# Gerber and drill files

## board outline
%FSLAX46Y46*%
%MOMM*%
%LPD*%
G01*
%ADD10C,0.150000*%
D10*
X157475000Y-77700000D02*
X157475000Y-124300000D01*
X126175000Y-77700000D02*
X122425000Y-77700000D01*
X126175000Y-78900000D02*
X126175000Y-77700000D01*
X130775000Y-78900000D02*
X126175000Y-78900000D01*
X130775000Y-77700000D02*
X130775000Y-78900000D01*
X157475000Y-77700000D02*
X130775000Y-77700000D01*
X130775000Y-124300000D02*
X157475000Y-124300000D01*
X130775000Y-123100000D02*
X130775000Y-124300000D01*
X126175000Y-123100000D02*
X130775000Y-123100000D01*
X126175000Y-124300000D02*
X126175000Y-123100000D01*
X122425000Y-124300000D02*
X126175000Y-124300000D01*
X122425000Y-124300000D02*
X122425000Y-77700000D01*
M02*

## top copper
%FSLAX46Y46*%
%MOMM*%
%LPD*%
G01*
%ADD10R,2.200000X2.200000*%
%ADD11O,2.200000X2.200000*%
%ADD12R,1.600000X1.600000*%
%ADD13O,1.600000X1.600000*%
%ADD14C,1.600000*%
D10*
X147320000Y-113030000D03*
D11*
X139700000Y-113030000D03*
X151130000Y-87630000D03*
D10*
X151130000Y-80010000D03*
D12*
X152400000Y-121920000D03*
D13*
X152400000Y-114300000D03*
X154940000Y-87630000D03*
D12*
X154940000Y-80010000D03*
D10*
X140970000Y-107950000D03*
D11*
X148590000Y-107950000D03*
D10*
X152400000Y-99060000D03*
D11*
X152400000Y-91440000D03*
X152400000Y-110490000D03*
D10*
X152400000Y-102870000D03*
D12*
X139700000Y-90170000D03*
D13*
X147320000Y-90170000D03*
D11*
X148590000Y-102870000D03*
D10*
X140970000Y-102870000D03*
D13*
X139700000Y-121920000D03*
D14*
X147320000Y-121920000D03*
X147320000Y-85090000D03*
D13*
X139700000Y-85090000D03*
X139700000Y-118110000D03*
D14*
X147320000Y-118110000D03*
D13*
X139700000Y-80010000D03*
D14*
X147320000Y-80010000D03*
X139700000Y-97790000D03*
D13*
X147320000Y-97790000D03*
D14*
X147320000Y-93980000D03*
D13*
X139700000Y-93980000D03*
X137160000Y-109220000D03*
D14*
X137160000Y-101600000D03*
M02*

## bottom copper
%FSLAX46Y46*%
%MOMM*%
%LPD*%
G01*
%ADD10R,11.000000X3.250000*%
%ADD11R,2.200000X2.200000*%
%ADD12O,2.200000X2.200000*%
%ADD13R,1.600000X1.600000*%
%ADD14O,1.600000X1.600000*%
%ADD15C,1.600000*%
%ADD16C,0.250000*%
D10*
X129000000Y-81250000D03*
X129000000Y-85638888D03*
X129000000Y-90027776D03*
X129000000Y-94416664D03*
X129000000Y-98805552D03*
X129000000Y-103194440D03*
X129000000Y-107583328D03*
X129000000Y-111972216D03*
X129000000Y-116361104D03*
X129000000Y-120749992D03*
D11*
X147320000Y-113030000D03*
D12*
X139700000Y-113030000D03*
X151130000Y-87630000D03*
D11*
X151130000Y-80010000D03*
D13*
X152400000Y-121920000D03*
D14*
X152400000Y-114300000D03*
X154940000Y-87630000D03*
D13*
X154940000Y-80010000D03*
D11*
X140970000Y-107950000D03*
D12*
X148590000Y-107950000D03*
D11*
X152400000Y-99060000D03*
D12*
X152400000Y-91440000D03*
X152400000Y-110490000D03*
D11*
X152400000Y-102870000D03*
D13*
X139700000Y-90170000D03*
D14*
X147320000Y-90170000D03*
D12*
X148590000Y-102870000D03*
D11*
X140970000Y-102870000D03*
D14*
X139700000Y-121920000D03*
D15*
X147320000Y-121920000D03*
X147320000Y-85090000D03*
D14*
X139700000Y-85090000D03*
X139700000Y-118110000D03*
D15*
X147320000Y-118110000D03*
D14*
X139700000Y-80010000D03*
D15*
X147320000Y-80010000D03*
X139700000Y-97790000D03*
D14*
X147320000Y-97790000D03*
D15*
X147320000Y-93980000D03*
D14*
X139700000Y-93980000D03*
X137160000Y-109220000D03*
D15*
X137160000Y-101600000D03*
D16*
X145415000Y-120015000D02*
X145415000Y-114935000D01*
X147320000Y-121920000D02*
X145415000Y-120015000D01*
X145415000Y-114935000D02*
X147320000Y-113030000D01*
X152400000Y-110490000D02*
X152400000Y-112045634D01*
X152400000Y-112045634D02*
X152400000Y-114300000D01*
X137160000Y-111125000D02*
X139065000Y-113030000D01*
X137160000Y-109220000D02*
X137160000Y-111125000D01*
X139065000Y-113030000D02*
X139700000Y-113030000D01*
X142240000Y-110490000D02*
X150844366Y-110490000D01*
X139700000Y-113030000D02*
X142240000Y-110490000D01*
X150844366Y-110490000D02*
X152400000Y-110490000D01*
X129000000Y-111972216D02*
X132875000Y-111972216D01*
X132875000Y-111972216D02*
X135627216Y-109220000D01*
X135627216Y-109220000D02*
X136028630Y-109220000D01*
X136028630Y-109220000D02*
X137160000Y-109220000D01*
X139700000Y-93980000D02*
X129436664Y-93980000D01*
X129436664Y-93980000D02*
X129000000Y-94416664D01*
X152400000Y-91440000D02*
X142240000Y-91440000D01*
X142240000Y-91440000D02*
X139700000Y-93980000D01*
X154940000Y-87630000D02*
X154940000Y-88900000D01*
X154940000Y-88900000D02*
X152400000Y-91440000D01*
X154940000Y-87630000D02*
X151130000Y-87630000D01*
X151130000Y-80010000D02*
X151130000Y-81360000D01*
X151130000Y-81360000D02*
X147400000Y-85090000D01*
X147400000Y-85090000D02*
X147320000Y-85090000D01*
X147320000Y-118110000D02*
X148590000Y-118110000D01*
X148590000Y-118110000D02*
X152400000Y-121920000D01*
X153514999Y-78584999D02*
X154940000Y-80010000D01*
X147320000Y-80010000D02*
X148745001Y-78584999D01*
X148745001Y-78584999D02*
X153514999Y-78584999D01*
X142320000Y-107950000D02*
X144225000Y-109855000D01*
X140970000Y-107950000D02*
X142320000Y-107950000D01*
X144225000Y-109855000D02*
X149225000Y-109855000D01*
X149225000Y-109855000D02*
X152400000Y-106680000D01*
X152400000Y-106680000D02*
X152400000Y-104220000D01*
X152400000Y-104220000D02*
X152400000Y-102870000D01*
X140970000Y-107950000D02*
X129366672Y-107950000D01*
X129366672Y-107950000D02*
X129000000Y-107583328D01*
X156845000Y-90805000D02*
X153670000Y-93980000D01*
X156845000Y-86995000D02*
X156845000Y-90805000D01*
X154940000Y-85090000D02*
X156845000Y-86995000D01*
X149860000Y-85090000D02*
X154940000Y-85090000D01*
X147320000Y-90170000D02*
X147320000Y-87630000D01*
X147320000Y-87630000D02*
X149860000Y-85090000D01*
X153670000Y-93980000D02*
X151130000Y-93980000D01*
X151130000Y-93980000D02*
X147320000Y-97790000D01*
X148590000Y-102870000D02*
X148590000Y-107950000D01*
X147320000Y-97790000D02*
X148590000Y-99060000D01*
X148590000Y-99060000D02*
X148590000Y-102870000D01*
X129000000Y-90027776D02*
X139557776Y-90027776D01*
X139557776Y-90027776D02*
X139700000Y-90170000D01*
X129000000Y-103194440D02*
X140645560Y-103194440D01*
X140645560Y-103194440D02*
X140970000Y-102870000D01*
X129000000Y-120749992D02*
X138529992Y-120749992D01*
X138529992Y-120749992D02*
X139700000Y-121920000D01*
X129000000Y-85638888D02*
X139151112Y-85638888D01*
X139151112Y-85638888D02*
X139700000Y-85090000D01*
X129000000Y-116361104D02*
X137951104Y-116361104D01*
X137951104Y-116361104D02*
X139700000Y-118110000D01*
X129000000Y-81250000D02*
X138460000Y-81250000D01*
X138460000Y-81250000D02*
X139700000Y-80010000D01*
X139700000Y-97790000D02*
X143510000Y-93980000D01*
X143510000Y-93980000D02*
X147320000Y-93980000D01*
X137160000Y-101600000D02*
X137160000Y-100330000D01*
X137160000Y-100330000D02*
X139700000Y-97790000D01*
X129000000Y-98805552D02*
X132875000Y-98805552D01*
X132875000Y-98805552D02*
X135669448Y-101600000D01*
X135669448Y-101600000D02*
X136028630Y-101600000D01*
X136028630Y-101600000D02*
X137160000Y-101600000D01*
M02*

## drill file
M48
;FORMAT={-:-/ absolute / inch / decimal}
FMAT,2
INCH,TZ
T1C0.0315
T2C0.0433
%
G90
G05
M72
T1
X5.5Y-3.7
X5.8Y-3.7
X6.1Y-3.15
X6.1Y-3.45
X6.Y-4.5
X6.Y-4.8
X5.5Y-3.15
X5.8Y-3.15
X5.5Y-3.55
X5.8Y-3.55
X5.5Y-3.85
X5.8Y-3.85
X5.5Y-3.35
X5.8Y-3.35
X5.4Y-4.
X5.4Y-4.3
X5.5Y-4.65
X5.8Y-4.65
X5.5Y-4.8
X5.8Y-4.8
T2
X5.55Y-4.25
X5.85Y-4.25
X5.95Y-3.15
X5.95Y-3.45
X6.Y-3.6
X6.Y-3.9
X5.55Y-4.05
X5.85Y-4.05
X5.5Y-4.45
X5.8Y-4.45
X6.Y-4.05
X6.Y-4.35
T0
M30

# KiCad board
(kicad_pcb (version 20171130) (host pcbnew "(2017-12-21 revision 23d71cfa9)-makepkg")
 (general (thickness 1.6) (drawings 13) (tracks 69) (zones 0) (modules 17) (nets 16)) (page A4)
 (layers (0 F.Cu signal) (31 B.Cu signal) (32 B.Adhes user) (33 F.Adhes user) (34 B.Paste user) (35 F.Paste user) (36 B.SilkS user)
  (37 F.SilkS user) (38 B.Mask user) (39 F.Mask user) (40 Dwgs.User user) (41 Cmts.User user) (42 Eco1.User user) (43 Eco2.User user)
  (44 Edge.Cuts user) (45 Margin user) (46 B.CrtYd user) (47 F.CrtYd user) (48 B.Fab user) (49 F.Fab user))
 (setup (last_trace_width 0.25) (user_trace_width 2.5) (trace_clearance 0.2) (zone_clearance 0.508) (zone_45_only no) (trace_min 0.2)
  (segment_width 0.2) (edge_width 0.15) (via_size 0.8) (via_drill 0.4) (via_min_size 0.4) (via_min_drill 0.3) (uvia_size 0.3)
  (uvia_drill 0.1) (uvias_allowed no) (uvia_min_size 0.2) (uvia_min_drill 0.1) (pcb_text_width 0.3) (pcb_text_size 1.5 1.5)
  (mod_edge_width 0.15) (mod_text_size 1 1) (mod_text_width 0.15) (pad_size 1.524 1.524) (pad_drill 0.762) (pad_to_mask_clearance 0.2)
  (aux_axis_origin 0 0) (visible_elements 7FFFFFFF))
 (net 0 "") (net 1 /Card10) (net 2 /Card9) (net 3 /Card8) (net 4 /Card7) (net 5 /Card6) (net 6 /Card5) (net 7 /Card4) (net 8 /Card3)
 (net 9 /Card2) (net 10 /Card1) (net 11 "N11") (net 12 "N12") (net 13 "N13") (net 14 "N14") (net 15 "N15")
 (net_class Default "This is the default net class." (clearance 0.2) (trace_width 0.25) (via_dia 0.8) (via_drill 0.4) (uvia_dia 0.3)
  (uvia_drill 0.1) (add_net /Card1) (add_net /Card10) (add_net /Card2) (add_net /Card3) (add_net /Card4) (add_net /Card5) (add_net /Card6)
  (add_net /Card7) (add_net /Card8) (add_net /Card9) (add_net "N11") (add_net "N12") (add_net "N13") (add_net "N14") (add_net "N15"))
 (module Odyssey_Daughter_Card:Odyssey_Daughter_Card (layer F.Cu) (at 129 101)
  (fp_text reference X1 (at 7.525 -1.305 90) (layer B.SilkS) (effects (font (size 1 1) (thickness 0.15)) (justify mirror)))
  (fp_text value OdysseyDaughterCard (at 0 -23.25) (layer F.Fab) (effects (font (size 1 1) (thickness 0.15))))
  (pad 10 smd rect (at 0 -19.75) (size 11 3.25) (layers B.Cu B.Mask) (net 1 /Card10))
  (pad 9 smd rect (at 0 -15.361112) (size 11 3.25) (layers B.Cu B.Mask) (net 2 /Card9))
  (pad 8 smd rect (at 0 -10.972224) (size 11 3.25) (layers B.Cu B.Mask) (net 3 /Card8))
  (pad 7 smd rect (at 0 -6.583336) (size 11 3.25) (layers B.Cu B.Mask) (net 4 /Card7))
  (pad 6 smd rect (at 0 -2.194448) (size 11 3.25) (layers B.Cu B.Mask) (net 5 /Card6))
  (pad 5 smd rect (at 0 2.19444) (size 11 3.25) (layers B.Cu B.Mask) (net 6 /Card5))
  (pad 4 smd rect (at 0 6.583328) (size 11 3.25) (layers B.Cu B.Mask) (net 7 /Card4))
  (pad 3 smd rect (at 0 10.972216) (size 11 3.25) (layers B.Cu B.Mask) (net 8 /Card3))
  (pad 2 smd rect (at 0 15.361104) (size 11 3.25) (layers B.Cu B.Mask) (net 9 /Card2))
  (pad 1 smd rect (at 0 19.749992) (size 11 3.25) (layers B.Cu B.Mask) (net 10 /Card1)))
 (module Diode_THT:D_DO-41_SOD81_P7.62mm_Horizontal (layer F.Cu) (at 147.32 113.03 180)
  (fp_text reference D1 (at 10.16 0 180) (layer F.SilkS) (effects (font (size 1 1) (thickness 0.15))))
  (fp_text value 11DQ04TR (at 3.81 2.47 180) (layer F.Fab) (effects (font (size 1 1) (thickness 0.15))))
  (pad 1 thru_hole rect (at 0 0 180) (size 2.2 2.2) (drill 1.1) (layers *.Cu *.Mask) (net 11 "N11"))
  (pad 2 thru_hole oval (at 7.62 0 180) (size 2.2 2.2) (drill 1.1) (layers *.Cu *.Mask) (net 8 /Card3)))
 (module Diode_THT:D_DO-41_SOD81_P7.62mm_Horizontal (layer F.Cu) (at 151.13 80.01 270)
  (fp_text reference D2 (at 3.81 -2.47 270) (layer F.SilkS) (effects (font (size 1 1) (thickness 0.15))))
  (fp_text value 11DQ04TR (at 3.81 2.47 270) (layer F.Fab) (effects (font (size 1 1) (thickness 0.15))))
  (pad 2 thru_hole oval (at 7.62 0 270) (size 2.2 2.2) (drill 1.1) (layers *.Cu *.Mask) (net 4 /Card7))
  (pad 1 thru_hole rect (at 0 0 270) (size 2.2 2.2) (drill 1.1) (layers *.Cu *.Mask) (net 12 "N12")))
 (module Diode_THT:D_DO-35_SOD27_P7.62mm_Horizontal (layer F.Cu) (at 152.4 121.92 90)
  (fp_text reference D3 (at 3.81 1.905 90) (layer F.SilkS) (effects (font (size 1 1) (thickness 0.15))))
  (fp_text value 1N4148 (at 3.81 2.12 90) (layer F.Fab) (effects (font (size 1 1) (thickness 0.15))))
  (pad 1 thru_hole rect (at 0 0 90) (size 1.6 1.6) (drill 0.8) (layers *.Cu *.Mask) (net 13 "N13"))
  (pad 2 thru_hole oval (at 7.62 0 90) (size 1.6 1.6) (drill 0.8) (layers *.Cu *.Mask) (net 8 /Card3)))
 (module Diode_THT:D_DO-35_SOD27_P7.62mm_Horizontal (layer F.Cu) (at 154.94 80.01 270)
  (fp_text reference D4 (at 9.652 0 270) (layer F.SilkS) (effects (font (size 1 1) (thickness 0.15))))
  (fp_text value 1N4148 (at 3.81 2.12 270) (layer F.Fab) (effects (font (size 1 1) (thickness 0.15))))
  (pad 2 thru_hole oval (at 7.62 0 270) (size 1.6 1.6) (drill 0.8) (layers *.Cu *.Mask) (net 4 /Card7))
  (pad 1 thru_hole rect (at 0 0 270) (size 1.6 1.6) (drill 0.8) (layers *.Cu *.Mask) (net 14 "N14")))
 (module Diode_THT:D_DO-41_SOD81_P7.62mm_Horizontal (layer F.Cu) (at 140.97 107.95)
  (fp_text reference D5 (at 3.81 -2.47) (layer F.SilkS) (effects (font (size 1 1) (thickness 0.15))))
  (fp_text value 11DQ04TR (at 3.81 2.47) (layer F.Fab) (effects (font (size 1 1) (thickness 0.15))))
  (pad 1 thru_hole rect (at 0 0) (size 2.2 2.2) (drill 1.1) (layers *.Cu *.Mask) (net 7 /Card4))
  (pad 2 thru_hole oval (at 7.62 0) (size 2.2 2.2) (drill 1.1) (layers *.Cu *.Mask) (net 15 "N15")))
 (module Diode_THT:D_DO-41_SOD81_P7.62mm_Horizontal (layer F.Cu) (at 152.4 99.06 90)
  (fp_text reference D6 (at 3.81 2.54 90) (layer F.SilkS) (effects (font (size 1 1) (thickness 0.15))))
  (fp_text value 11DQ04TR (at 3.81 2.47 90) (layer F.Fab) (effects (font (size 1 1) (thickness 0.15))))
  (pad 1 thru_hole rect (at 0 0 90) (size 2.2 2.2) (drill 1.1) (layers *.Cu *.Mask) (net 7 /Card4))
  (pad 2 thru_hole oval (at 7.62 0 90) (size 2.2 2.2) (drill 1.1) (layers *.Cu *.Mask) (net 4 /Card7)))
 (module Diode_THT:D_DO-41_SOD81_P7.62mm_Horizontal (layer F.Cu) (at 152.4 102.87 270)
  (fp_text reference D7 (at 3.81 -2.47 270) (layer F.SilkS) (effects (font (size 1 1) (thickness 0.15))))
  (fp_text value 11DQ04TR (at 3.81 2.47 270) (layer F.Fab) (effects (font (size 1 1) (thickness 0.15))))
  (pad 2 thru_hole oval (at 7.62 0 270) (size 2.2 2.2) (drill 1.1) (layers *.Cu *.Mask) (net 8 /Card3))
  (pad 1 thru_hole rect (at 0 0 270) (size 2.2 2.2) (drill 1.1) (layers *.Cu *.Mask) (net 7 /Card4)))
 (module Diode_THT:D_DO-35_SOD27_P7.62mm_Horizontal (layer F.Cu) (at 139.7 90.17)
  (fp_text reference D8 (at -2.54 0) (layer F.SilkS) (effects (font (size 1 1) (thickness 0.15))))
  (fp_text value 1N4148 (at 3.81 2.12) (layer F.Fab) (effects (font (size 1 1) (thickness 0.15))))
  (pad 1 thru_hole rect (at 0 0) (size 1.6 1.6) (drill 0.8) (layers *.Cu *.Mask) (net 3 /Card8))
  (pad 2 thru_hole oval (at 7.62 0) (size 1.6 1.6) (drill 0.8) (layers *.Cu *.Mask) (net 15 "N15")))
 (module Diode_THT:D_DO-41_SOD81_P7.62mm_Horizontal (layer F.Cu) (at 140.97 102.87)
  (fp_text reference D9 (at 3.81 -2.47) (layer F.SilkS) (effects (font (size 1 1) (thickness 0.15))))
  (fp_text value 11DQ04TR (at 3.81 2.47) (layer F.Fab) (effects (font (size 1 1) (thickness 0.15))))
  (pad 2 thru_hole oval (at 7.62 0) (size 2.2 2.2) (drill 1.1) (layers *.Cu *.Mask) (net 15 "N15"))
  (pad 1 thru_hole rect (at 0 0) (size 2.2 2.2) (drill 1.1) (layers *.Cu *.Mask) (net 6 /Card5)))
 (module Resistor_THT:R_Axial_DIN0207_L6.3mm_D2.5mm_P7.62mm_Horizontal (layer F.Cu) (at 147.32 121.92 180)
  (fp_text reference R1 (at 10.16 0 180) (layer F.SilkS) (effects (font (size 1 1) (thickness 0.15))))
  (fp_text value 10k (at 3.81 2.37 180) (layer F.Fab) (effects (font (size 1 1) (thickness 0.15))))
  (pad 2 thru_hole oval (at 7.62 0 180) (size 1.6 1.6) (drill 0.8) (layers *.Cu *.Mask) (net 10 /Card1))
  (pad 1 thru_hole circle (at 0 0 180) (size 1.6 1.6) (drill 0.8) (layers *.Cu *.Mask) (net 11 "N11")))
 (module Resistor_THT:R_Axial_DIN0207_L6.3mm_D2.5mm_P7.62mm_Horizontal (layer F.Cu) (at 147.32 85.09 180)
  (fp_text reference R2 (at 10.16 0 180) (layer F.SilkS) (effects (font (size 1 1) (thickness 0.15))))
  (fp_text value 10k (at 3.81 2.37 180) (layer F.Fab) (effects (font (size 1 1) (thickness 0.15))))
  (pad 1 thru_hole circle (at 0 0 180) (size 1.6 1.6) (drill 0.8) (layers *.Cu *.Mask) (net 12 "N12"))
  (pad 2 thru_hole oval (at 7.62 0 180) (size 1.6 1.6) (drill 0.8) (layers *.Cu *.Mask) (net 2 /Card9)))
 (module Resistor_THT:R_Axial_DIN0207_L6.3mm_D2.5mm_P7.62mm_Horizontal (layer F.Cu) (at 147.32 118.11 180)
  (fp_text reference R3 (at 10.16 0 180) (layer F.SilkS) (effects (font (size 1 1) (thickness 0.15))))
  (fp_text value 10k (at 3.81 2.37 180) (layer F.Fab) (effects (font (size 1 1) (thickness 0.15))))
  (pad 2 thru_hole oval (at 7.62 0 180) (size 1.6 1.6) (drill 0.8) (layers *.Cu *.Mask) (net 9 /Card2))
  (pad 1 thru_hole circle (at 0 0 180) (size 1.6 1.6) (drill 0.8) (layers *.Cu *.Mask) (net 13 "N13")))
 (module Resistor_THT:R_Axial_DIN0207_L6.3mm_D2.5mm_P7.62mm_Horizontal (layer F.Cu) (at 147.32 80.01 180)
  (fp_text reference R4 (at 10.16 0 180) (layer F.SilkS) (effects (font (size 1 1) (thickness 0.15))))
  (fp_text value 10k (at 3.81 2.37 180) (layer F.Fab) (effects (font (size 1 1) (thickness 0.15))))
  (pad 2 thru_hole oval (at 7.62 0 180) (size 1.6 1.6) (drill 0.8) (layers *.Cu *.Mask) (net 1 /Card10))
  (pad 1 thru_hole circle (at 0 0 180) (size 1.6 1.6) (drill 0.8) (layers *.Cu *.Mask) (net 14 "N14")))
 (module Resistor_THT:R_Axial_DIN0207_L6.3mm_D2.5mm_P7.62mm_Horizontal (layer F.Cu) (at 139.7 97.79)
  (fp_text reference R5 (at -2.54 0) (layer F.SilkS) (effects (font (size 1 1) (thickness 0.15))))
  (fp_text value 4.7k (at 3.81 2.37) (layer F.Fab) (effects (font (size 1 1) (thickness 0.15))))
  (pad 1 thru_hole circle (at 0 0) (size 1.6 1.6) (drill 0.8) (layers *.Cu *.Mask) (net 5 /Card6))
  (pad 2 thru_hole oval (at 7.62 0) (size 1.6 1.6) (drill 0.8) (layers *.Cu *.Mask) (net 15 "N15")))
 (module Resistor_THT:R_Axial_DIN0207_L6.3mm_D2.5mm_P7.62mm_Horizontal (layer F.Cu) (at 147.32 93.98 180)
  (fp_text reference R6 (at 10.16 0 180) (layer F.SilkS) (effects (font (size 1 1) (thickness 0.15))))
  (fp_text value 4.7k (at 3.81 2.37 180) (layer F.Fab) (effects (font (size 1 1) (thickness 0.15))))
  (pad 1 thru_hole circle (at 0 0 180) (size 1.6 1.6) (drill 0.8) (layers *.Cu *.Mask) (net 5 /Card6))
  (pad 2 thru_hole oval (at 7.62 0 180) (size 1.6 1.6) (drill 0.8) (layers *.Cu *.Mask) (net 4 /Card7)))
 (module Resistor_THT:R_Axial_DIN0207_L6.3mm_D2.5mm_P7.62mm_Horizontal (layer F.Cu) (at 137.16 101.6 270)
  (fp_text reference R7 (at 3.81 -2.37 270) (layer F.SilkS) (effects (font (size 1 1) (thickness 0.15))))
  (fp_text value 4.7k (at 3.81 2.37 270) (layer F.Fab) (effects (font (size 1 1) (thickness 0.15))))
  (pad 2 thru_hole oval (at 7.62 0 270) (size 1.6 1.6) (drill 0.8) (layers *.Cu *.Mask) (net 8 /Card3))
  (pad 1 thru_hole circle (at 0 0 270) (size 1.6 1.6) (drill 0.8) (layers *.Cu *.Mask) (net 5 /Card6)))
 (gr_line (start 157.475 77.7) (end 157.475 124.3) (layer Edge.Cuts) (width 0.15))
 (gr_line (start 126.175 77.7) (end 122.425 77.7) (layer Edge.Cuts) (width 0.15))
 (gr_line (start 126.175 78.9) (end 126.175 77.7) (layer Edge.Cuts) (width 0.15))
 (gr_line (start 130.775 78.9) (end 126.175 78.9) (layer Edge.Cuts) (width 0.15))
 (gr_line (start 130.775 77.7) (end 130.775 78.9) (layer Edge.Cuts) (width 0.15))
 (gr_line (start 157.475 77.7) (end 130.775 77.7) (layer Edge.Cuts) (width 0.15))
 (gr_line (start 130.775 124.3) (end 157.475 124.3) (layer Edge.Cuts) (width 0.15))
 (gr_line (start 130.775 123.1) (end 130.775 124.3) (layer Edge.Cuts) (width 0.15))
 (gr_line (start 126.175 123.1) (end 130.775 123.1) (layer Edge.Cuts) (width 0.15))
 (gr_line (start 126.175 124.3) (end 126.175 123.1) (layer Edge.Cuts) (width 0.15))
 (gr_line (start 122.425 124.3) (end 126.175 124.3) (layer Edge.Cuts) (width 0.15))
 (gr_line (start 122.425 124.3) (end 122.425 77.7) (layer Edge.Cuts) (width 0.15))
 (segment (start 145.415 120.015) (end 145.415 114.935) (width 0.25) (layer B.Cu) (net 11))
 (segment (start 147.32 121.92) (end 145.415 120.015) (width 0.25) (layer B.Cu) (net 11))
 (segment (start 145.415 114.935) (end 147.32 113.03) (width 0.25) (layer B.Cu) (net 11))
 (segment (start 152.4 110.49) (end 152.4 112.045634) (width 0.25) (layer B.Cu) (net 8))
 (segment (start 152.4 112.045634) (end 152.4 114.3) (width 0.25) (layer B.Cu) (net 8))
 (segment (start 137.16 111.125) (end 139.065 113.03) (width 0.25) (layer B.Cu) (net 8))
 (segment (start 137.16 109.22) (end 137.16 111.125) (width 0.25) (layer B.Cu) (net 8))
 (segment (start 139.065 113.03) (end 139.7 113.03) (width 0.25) (layer B.Cu) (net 8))
 (segment (start 142.24 110.49) (end 150.844366 110.49) (width 0.25) (layer B.Cu) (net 8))
 (segment (start 139.7 113.03) (end 142.24 110.49) (width 0.25) (layer B.Cu) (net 8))
 (segment (start 150.844366 110.49) (end 152.4 110.49) (width 0.25) (layer B.Cu) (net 8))
 (segment (start 129 111.972216) (end 132.875 111.972216) (width 0.25) (layer B.Cu) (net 8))
 (segment (start 132.875 111.972216) (end 135.627216 109.22) (width 0.25) (layer B.Cu) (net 8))
 (segment (start 135.627216 109.22) (end 136.02863 109.22) (width 0.25) (layer B.Cu) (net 8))
 (segment (start 136.02863 109.22) (end 137.16 109.22) (width 0.25) (layer B.Cu) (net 8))
 (segment (start 139.7 93.98) (end 129.436664 93.98) (width 0.25) (layer B.Cu) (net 4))
 (segment (start 129.436664 93.98) (end 129 94.416664) (width 0.25) (layer B.Cu) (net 4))
 (segment (start 152.4 91.44) (end 142.24 91.44) (width 0.25) (layer B.Cu) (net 4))
 (segment (start 142.24 91.44) (end 139.7 93.98) (width 0.25) (layer B.Cu) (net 4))
 (segment (start 154.94 87.63) (end 154.94 88.9) (width 0.25) (layer B.Cu) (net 4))
 (segment (start 154.94 88.9) (end 152.4 91.44) (width 0.25) (layer B.Cu) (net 4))
 (segment (start 154.94 87.63) (end 151.13 87.63) (width 0.25) (layer B.Cu) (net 4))
 (segment (start 151.13 80.01) (end 151.13 81.36) (width 0.25) (layer B.Cu) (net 12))
 (segment (start 151.13 81.36) (end 147.4 85.09) (width 0.25) (layer B.Cu) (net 12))
 (segment (start 147.4 85.09) (end 147.32 85.09) (width 0.25) (layer B.Cu) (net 12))
 (segment (start 147.32 118.11) (end 148.59 118.11) (width 0.25) (layer B.Cu) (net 13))
 (segment (start 148.59 118.11) (end 152.4 121.92) (width 0.25) (layer B.Cu) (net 13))
 (segment (start 153.514999 78.584999) (end 154.94 80.01) (width 0.25) (layer B.Cu) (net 14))
 (segment (start 147.32 80.01) (end 148.745001 78.584999) (width 0.25) (layer B.Cu) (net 14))
 (segment (start 148.745001 78.584999) (end 153.514999 78.584999) (width 0.25) (layer B.Cu) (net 14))
 (segment (start 142.32 107.95) (end 144.225 109.855) (width 0.25) (layer B.Cu) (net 7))
 (segment (start 140.97 107.95) (end 142.32 107.95) (width 0.25) (layer B.Cu) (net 7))
 (segment (start 144.225 109.855) (end 149.225 109.855) (width 0.25) (layer B.Cu) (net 7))
 (segment (start 149.225 109.855) (end 152.4 106.68) (width 0.25) (layer B.Cu) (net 7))
 (segment (start 152.4 106.68) (end 152.4 104.22) (width 0.25) (layer B.Cu) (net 7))
 (segment (start 152.4 104.22) (end 152.4 102.87) (width 0.25) (layer B.Cu) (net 7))
 (segment (start 140.97 107.95) (end 129.366672 107.95) (width 0.25) (layer B.Cu) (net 7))
 (segment (start 129.366672 107.95) (end 129 107.583328) (width 0.25) (layer B.Cu) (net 7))
 (segment (start 156.845 90.805) (end 153.67 93.98) (width 0.25) (layer B.Cu) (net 15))
 (segment (start 156.845 86.995) (end 156.845 90.805) (width 0.25) (layer B.Cu) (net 15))
 (segment (start 154.94 85.09) (end 156.845 86.995) (width 0.25) (layer B.Cu) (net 15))
 (segment (start 149.86 85.09) (end 154.94 85.09) (width 0.25) (layer B.Cu) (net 15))
 (segment (start 147.32 90.17) (end 147.32 87.63) (width 0.25) (layer B.Cu) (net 15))
 (segment (start 147.32 87.63) (end 149.86 85.09) (width 0.25) (layer B.Cu) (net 15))
 (segment (start 153.67 93.98) (end 151.13 93.98) (width 0.25) (layer B.Cu) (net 15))
 (segment (start 151.13 93.98) (end 147.32 97.79) (width 0.25) (layer B.Cu) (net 15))
 (segment (start 148.59 102.87) (end 148.59 107.95) (width 0.25) (layer B.Cu) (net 15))
 (segment (start 147.32 97.79) (end 148.59 99.06) (width 0.25) (layer B.Cu) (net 15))
 (segment (start 148.59 99.06) (end 148.59 102.87) (width 0.25) (layer B.Cu) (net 15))
 (segment (start 129 90.027776) (end 139.557776 90.027776) (width 0.25) (layer B.Cu) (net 3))
 (segment (start 139.557776 90.027776) (end 139.7 90.17) (width 0.25) (layer B.Cu) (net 3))
 (segment (start 129 103.19444) (end 140.64556 103.19444) (width 0.25) (layer B.Cu) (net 6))
 (segment (start 140.64556 103.19444) (end 140.97 102.87) (width 0.25) (layer B.Cu) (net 6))
 (segment (start 129 120.749992) (end 138.529992 120.749992) (width 0.25) (layer B.Cu) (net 10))
 (segment (start 138.529992 120.749992) (end 139.7 121.92) (width 0.25) (layer B.Cu) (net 10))
 (segment (start 129 85.638888) (end 139.151112 85.638888) (width 0.25) (layer B.Cu) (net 2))
 (segment (start 139.151112 85.638888) (end 139.7 85.09) (width 0.25) (layer B.Cu) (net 2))
 (segment (start 129 116.361104) (end 137.951104 116.361104) (width 0.25) (layer B.Cu) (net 9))
 (segment (start 137.951104 116.361104) (end 139.7 118.11) (width 0.25) (layer B.Cu) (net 9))
 (segment (start 129 81.25) (end 138.46 81.25) (width 0.25) (layer B.Cu) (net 1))
 (segment (start 138.46 81.25) (end 139.7 80.01) (width 0.25) (layer B.Cu) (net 1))
 (segment (start 139.7 97.79) (end 143.51 93.98) (width 0.25) (layer B.Cu) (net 5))
 (segment (start 143.51 93.98) (end 147.32 93.98) (width 0.25) (layer B.Cu) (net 5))
 (segment (start 137.16 101.6) (end 137.16 100.33) (width 0.25) (layer B.Cu) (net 5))
 (segment (start 137.16 100.33) (end 139.7 97.79) (width 0.25) (layer B.Cu) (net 5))
 (segment (start 129 98.805552) (end 132.875 98.805552) (width 0.25) (layer B.Cu) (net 5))
 (segment (start 132.875 98.805552) (end 135.669448 101.6) (width 0.25) (layer B.Cu) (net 5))
 (segment (start 135.669448 101.6) (end 136.02863 101.6) (width 0.25) (layer B.Cu) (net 5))
 (segment (start 136.02863 101.6) (end 137.16 101.6) (width 0.25) (layer B.Cu) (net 5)))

